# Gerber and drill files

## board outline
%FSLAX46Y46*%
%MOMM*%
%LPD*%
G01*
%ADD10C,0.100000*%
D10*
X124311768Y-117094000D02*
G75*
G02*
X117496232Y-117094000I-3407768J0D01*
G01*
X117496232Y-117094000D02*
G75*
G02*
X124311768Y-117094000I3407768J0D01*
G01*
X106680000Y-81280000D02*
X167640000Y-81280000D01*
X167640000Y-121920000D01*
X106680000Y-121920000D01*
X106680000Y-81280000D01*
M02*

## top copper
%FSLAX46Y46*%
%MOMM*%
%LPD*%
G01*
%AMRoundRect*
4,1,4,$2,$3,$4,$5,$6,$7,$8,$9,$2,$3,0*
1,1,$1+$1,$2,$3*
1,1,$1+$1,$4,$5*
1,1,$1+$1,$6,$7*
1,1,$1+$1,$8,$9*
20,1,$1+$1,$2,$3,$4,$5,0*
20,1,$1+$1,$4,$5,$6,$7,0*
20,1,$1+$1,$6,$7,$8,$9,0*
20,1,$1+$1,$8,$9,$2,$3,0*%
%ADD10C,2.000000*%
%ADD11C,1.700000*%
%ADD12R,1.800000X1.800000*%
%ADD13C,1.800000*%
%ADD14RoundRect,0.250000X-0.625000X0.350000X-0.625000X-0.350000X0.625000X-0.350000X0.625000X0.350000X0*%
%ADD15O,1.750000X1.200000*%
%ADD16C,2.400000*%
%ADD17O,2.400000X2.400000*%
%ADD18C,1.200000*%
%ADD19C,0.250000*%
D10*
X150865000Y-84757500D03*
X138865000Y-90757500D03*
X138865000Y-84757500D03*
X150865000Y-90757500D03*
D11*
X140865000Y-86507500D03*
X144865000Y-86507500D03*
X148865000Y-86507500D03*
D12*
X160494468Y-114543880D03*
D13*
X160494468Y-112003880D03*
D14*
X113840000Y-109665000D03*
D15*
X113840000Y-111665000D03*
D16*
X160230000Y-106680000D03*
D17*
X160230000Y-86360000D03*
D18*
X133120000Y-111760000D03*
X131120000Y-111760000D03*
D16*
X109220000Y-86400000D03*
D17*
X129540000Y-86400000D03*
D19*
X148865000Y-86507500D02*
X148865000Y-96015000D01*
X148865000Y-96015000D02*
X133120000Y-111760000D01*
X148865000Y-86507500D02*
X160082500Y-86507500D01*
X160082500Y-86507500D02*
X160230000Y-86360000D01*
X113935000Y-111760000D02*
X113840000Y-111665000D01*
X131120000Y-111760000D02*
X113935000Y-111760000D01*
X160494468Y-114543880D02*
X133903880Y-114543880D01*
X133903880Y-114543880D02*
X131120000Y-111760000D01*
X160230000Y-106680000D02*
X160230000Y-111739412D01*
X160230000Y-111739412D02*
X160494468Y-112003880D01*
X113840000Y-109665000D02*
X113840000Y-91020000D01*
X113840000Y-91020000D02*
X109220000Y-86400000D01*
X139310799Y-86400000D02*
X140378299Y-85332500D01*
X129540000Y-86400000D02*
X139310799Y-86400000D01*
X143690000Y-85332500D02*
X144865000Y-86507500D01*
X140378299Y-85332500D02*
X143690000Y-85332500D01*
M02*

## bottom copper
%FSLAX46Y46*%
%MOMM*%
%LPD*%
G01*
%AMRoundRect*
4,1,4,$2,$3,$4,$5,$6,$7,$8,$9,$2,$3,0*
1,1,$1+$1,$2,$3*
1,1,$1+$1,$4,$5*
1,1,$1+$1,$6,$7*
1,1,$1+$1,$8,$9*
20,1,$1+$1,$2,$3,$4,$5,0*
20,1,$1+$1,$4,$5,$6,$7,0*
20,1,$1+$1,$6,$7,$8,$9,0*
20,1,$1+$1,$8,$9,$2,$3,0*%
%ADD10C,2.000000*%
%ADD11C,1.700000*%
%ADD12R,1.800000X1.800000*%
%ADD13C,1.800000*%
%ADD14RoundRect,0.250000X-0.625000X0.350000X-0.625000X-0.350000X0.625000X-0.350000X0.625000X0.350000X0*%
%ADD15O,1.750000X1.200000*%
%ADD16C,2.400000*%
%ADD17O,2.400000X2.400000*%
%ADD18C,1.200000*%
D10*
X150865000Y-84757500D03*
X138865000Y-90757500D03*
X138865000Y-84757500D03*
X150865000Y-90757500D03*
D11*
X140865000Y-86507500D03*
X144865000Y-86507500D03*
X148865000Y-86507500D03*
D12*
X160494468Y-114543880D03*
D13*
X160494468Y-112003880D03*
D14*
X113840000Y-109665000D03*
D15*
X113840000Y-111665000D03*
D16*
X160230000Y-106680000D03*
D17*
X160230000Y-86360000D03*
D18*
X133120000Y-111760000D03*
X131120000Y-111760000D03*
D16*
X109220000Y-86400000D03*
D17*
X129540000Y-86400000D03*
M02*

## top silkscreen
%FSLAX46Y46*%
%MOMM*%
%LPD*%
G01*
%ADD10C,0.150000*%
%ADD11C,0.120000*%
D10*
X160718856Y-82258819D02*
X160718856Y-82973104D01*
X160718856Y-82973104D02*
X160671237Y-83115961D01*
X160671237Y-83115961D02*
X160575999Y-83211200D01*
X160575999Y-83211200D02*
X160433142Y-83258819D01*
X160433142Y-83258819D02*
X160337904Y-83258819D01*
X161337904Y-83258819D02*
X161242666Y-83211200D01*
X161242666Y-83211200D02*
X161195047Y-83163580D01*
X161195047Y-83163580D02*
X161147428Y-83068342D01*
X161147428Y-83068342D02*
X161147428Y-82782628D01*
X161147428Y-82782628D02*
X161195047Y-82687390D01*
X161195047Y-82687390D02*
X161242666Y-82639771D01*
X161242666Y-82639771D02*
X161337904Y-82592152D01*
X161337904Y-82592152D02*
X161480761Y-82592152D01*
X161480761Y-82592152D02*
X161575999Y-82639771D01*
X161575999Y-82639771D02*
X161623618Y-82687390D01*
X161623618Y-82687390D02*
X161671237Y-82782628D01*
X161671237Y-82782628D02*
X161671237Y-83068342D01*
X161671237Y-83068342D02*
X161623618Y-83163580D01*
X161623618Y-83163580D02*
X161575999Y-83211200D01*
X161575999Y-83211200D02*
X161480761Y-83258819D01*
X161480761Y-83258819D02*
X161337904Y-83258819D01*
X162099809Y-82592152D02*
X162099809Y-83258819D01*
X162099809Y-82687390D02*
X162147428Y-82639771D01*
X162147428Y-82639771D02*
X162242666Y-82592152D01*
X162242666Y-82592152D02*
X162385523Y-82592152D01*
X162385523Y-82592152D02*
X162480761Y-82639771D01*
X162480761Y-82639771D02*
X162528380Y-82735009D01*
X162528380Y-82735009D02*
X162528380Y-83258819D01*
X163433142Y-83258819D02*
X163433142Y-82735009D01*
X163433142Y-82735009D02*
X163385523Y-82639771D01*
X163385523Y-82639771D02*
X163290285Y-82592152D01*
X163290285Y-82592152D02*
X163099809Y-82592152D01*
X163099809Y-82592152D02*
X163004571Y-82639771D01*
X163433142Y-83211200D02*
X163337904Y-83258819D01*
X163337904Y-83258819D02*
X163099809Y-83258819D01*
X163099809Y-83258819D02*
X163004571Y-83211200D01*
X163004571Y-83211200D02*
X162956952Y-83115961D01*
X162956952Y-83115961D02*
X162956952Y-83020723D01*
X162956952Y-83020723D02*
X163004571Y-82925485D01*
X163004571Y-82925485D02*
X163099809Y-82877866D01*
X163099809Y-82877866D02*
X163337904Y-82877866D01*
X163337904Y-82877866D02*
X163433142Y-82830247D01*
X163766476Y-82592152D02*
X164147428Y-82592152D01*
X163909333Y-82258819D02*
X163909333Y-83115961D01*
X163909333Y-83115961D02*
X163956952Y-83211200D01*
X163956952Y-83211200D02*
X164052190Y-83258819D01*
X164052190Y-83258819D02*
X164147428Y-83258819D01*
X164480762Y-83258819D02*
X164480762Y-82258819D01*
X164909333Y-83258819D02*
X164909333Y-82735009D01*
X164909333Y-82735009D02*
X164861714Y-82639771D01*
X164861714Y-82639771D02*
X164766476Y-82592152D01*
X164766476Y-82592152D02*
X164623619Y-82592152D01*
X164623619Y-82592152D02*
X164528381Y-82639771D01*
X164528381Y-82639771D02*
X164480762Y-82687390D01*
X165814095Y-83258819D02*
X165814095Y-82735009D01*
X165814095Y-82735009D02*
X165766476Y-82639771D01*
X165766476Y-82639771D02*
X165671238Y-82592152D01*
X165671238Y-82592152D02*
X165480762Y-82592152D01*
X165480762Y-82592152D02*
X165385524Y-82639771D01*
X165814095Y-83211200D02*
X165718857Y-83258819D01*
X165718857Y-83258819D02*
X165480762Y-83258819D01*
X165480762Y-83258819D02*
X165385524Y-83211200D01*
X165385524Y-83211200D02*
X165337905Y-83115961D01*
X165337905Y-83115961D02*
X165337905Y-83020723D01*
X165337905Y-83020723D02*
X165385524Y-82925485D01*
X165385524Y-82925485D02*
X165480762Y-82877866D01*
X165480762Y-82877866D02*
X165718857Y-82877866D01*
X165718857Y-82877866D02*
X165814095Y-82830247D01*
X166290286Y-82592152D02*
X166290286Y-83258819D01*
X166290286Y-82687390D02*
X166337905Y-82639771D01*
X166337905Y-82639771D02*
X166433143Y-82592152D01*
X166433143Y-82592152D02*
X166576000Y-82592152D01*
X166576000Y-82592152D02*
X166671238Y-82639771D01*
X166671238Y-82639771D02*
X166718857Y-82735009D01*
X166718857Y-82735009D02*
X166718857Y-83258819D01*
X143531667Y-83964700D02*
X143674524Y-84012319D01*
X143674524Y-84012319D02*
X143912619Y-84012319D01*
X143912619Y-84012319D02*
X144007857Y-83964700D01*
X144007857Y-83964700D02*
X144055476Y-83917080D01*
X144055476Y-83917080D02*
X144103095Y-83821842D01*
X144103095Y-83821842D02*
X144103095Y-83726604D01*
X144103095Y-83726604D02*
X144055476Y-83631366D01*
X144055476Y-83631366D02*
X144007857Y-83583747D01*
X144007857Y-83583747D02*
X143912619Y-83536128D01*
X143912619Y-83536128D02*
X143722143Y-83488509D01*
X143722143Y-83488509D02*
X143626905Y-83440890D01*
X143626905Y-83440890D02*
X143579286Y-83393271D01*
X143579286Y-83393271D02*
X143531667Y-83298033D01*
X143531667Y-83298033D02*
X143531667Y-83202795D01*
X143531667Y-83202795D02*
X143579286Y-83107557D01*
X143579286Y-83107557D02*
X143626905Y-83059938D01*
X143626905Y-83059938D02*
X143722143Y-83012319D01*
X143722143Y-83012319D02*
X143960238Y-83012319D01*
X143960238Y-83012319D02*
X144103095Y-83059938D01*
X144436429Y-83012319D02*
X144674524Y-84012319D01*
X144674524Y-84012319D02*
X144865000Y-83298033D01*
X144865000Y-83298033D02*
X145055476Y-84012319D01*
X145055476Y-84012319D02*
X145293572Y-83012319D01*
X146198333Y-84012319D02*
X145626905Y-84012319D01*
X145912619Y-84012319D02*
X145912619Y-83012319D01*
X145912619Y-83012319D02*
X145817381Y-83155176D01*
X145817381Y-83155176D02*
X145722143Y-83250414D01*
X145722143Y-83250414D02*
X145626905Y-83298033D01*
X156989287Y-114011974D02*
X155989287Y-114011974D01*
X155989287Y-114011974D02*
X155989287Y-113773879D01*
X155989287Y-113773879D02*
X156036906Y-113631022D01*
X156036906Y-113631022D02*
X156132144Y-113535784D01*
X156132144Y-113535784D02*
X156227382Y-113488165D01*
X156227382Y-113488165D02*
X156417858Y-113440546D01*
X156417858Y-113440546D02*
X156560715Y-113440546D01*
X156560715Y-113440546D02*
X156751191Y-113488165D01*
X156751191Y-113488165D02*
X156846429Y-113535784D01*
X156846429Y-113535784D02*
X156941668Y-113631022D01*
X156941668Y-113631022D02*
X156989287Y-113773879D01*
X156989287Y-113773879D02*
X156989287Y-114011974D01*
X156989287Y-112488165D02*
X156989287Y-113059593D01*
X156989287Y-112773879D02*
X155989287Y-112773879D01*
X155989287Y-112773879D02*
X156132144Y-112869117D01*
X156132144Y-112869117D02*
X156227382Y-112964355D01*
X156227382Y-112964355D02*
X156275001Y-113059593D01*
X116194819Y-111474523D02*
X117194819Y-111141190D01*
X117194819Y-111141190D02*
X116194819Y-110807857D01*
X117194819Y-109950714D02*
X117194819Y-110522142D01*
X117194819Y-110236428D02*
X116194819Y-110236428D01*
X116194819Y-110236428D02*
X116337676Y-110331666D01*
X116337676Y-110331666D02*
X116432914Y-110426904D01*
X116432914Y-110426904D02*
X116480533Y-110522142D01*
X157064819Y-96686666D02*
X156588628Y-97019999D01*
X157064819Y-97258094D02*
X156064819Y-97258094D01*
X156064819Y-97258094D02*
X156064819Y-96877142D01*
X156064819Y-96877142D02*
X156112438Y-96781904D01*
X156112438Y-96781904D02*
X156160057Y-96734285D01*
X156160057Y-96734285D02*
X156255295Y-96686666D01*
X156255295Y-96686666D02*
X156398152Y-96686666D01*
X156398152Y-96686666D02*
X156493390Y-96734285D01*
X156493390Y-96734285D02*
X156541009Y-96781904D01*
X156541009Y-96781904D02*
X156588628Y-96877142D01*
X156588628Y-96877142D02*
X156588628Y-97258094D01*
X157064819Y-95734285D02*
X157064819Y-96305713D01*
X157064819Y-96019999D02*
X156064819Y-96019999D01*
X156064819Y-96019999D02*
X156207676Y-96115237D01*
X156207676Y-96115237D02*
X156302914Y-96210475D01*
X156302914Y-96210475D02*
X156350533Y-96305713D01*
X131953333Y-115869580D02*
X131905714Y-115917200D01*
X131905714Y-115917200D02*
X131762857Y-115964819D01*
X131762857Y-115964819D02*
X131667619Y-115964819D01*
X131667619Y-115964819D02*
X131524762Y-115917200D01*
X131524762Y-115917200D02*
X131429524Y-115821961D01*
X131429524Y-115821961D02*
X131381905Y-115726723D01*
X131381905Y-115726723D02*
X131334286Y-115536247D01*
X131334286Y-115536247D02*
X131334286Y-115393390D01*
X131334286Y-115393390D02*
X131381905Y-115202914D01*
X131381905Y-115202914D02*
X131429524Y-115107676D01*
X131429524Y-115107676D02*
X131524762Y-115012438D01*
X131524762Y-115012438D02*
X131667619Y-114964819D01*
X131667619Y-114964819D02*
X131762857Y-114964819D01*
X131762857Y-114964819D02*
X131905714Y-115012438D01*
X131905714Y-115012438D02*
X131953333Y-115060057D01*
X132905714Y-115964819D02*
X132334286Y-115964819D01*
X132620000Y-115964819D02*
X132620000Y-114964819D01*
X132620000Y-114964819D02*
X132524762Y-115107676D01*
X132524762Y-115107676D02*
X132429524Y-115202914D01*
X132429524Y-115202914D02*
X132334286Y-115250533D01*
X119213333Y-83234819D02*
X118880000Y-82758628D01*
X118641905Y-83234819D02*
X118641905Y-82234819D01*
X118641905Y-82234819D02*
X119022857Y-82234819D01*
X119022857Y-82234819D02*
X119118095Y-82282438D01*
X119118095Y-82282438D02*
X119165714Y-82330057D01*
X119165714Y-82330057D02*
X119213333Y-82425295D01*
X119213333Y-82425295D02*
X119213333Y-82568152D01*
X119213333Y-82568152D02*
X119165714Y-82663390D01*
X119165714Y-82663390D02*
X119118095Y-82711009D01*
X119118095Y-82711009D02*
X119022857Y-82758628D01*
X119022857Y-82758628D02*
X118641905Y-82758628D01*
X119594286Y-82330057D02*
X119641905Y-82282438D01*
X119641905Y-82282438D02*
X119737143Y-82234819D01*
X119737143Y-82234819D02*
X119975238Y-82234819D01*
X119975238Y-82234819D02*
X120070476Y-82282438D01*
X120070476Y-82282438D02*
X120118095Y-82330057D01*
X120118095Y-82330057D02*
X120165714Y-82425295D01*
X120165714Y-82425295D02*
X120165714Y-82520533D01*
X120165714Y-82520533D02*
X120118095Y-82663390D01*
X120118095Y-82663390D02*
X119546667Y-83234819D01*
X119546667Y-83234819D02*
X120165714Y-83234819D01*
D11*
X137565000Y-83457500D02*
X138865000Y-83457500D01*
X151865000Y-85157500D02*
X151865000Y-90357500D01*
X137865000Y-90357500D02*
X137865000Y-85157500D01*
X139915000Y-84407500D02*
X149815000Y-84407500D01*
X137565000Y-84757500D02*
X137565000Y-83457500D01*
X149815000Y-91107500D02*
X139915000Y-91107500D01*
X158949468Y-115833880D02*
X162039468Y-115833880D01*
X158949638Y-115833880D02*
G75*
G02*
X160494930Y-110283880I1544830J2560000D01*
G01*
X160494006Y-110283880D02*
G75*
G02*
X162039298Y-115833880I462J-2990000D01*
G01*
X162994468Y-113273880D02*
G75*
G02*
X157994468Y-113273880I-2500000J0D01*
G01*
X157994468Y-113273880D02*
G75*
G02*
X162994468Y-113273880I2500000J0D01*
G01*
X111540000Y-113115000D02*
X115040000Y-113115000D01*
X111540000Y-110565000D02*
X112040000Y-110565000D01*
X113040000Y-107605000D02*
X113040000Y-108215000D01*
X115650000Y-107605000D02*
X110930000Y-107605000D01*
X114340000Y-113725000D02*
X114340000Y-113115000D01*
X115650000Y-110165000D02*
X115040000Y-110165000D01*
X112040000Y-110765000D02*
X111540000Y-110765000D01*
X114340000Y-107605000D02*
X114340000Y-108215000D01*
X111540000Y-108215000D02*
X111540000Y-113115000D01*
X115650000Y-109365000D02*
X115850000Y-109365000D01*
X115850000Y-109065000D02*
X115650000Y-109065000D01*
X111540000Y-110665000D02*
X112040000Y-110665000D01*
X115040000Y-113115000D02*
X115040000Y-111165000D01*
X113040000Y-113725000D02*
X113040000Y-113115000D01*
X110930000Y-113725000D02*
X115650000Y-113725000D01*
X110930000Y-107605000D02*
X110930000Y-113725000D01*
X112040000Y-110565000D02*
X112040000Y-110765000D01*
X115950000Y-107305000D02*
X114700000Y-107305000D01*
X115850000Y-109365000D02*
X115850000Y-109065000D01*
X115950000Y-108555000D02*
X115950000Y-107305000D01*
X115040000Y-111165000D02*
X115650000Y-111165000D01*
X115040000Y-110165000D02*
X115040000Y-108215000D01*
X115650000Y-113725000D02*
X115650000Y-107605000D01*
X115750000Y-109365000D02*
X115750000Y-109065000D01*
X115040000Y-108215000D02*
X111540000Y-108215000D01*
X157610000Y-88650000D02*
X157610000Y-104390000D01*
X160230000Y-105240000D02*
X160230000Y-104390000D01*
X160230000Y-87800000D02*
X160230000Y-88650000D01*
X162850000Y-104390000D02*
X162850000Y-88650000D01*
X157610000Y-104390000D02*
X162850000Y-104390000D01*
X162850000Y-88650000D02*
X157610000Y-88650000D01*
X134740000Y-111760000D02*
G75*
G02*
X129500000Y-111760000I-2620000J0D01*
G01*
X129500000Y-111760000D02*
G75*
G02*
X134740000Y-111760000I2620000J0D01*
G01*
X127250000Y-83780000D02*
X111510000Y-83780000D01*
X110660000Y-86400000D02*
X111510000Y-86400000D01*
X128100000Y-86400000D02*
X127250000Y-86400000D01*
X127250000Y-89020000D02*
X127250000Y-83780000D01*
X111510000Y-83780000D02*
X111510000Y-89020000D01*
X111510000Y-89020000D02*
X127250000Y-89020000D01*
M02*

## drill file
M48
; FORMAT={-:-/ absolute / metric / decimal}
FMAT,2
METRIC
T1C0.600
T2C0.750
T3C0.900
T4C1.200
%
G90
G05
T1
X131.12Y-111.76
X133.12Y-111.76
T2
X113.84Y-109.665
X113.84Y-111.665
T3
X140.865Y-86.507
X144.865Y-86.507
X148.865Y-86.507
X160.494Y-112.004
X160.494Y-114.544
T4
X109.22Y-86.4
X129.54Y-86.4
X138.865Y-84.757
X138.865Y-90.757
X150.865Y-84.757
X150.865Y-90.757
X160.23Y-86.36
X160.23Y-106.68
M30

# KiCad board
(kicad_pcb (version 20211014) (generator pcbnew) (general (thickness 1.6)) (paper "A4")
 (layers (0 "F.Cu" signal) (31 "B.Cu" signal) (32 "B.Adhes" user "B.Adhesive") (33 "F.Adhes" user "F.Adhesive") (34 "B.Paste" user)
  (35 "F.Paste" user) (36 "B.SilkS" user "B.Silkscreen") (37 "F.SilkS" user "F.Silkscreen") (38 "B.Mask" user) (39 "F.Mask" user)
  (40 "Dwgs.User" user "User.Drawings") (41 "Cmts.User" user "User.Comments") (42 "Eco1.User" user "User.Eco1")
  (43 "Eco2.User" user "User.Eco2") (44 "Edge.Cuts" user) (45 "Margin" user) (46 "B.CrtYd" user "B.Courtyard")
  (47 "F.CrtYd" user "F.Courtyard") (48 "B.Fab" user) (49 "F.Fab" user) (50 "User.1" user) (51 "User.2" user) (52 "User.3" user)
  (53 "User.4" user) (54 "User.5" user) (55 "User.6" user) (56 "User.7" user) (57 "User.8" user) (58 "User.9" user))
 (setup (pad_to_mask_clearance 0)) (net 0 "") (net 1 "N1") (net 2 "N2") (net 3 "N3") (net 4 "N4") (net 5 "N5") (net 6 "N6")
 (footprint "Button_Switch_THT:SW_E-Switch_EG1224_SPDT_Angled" (layer "F.Cu") (at 140.865 86.5075)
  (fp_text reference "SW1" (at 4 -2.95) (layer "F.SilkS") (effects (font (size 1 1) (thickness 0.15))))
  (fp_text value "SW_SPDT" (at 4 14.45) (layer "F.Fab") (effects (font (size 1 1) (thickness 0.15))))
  (fp_line (start -3.3 -3.05) (end -2 -3.05) (layer "F.SilkS") (width 0.12))
  (fp_line (start 11 -1.35) (end 11 3.85) (layer "F.SilkS") (width 0.12))
  (fp_line (start -3 3.85) (end -3 -1.35) (layer "F.SilkS") (width 0.12))
  (fp_line (start -0.95 -2.1) (end 8.95 -2.1) (layer "F.SilkS") (width 0.12))
  (fp_line (start -3.3 -1.75) (end -3.3 -3.05) (layer "F.SilkS") (width 0.12))
  (fp_line (start 8.95 4.6) (end -0.95 4.6) (layer "F.SilkS") (width 0.12))
  (pad "" thru_hole circle (at 10 -1.75) (size 2 2) (drill 1.2) (layers *.Cu *.Mask))
  (pad "" thru_hole circle (at -2 4.25) (size 2 2) (drill 1.2) (layers *.Cu *.Mask))
  (pad "" thru_hole circle (at -2 -1.75) (size 2 2) (drill 1.2) (layers *.Cu *.Mask))
  (pad "" thru_hole circle (at 10 4.25) (size 2 2) (drill 1.2) (layers *.Cu *.Mask))
  (pad "1" thru_hole circle (at 0 0) (size 1.7 1.7) (drill 0.9) (layers *.Cu *.Mask) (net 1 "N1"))
  (pad "2" thru_hole circle (at 4 0) (size 1.7 1.7) (drill 0.9) (layers *.Cu *.Mask) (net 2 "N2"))
  (pad "3" thru_hole circle (at 8 0) (size 1.7 1.7) (drill 0.9) (layers *.Cu *.Mask) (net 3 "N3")))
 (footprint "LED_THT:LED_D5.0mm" (layer "F.Cu") (at 160.494468 114.54388 90)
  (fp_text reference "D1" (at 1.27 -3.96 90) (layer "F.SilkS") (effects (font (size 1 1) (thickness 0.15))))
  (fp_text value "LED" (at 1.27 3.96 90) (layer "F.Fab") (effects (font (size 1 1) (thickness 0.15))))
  (fp_line (start -1.29 -1.545) (end -1.29 1.545) (layer "F.SilkS") (width 0.12))
  (fp_arc (start -1.29 -1.54483) (mid 2.072002 -2.880433) (end 4.26 0.000462) (layer "F.SilkS") (width 0.12))
  (fp_arc (start 4.26 -0.000462) (mid 2.072002 2.880433) (end -1.29 1.54483) (layer "F.SilkS") (width 0.12))
  (fp_circle (center 1.27 0) (end 3.77 0) (layer "F.SilkS") (width 0.12) (fill none))
  (pad "1" thru_hole rect (at 0 0 90) (size 1.8 1.8) (drill 0.9) (layers *.Cu *.Mask) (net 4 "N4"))
  (pad "2" thru_hole circle (at 2.54 0 90) (size 1.8 1.8) (drill 0.9) (layers *.Cu *.Mask) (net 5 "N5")))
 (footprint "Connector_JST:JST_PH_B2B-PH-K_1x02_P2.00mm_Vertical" (layer "F.Cu") (at 113.84 109.665 -90)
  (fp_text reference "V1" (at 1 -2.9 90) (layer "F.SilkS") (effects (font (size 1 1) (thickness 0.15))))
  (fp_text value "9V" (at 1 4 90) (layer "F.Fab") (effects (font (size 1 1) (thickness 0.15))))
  (fp_line (start 3.45 2.3) (end 3.45 -1.2) (layer "F.SilkS") (width 0.12))
  (fp_line (start 0.9 2.3) (end 0.9 1.8) (layer "F.SilkS") (width 0.12))
  (fp_line (start -2.06 0.8) (end -1.45 0.8) (layer "F.SilkS") (width 0.12))
  (fp_line (start -2.06 -1.81) (end -2.06 2.91) (layer "F.SilkS") (width 0.12))
  (fp_line (start 4.06 -0.5) (end 3.45 -0.5) (layer "F.SilkS") (width 0.12))
  (fp_line (start 0.5 -1.81) (end 0.5 -1.2) (layer "F.SilkS") (width 0.12))
  (fp_line (start 1.1 1.8) (end 1.1 2.3) (layer "F.SilkS") (width 0.12))
  (fp_line (start -2.06 -0.5) (end -1.45 -0.5) (layer "F.SilkS") (width 0.12))
  (fp_line (start -1.45 2.3) (end 3.45 2.3) (layer "F.SilkS") (width 0.12))
  (fp_line (start -0.3 -1.81) (end -0.3 -2.01) (layer "F.SilkS") (width 0.12))
  (fp_line (start -0.6 -2.01) (end -0.6 -1.81) (layer "F.SilkS") (width 0.12))
  (fp_line (start 1 2.3) (end 1 1.8) (layer "F.SilkS") (width 0.12))
  (fp_line (start 3.45 -1.2) (end 1.5 -1.2) (layer "F.SilkS") (width 0.12))
  (fp_line (start 4.06 0.8) (end 3.45 0.8) (layer "F.SilkS") (width 0.12))
  (fp_line (start 4.06 2.91) (end 4.06 -1.81) (layer "F.SilkS") (width 0.12))
  (fp_line (start -2.06 2.91) (end 4.06 2.91) (layer "F.SilkS") (width 0.12))
  (fp_line (start 0.9 1.8) (end 1.1 1.8) (layer "F.SilkS") (width 0.12))
  (fp_line (start -2.36 -2.11) (end -2.36 -0.86) (layer "F.SilkS") (width 0.12))
  (fp_line (start -0.3 -2.01) (end -0.6 -2.01) (layer "F.SilkS") (width 0.12))
  (fp_line (start -1.11 -2.11) (end -2.36 -2.11) (layer "F.SilkS") (width 0.12))
  (fp_line (start 1.5 -1.2) (end 1.5 -1.81) (layer "F.SilkS") (width 0.12))
  (fp_line (start 0.5 -1.2) (end -1.45 -1.2) (layer "F.SilkS") (width 0.12))
  (fp_line (start 4.06 -1.81) (end -2.06 -1.81) (layer "F.SilkS") (width 0.12))
  (fp_line (start -0.3 -1.91) (end -0.6 -1.91) (layer "F.SilkS") (width 0.12))
  (fp_line (start -1.45 -1.2) (end -1.45 2.3) (layer "F.SilkS") (width 0.12))
  (pad "1" thru_hole roundrect (at 0 0 270) (size 1.2 1.75) (drill 0.75) (layers *.Cu *.Mask) (roundrect_rratio 0.208333) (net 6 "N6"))
  (pad "2" thru_hole oval (at 2 0 270) (size 1.2 1.75) (drill 0.75) (layers *.Cu *.Mask) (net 4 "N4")))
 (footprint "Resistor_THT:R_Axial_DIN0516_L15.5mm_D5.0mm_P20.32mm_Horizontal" (layer "F.Cu") (at 160.23 106.68 90)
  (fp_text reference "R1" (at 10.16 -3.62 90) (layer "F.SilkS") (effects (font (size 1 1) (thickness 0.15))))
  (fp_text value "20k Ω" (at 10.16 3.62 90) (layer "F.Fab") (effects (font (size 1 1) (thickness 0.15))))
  (fp_line (start 18.03 -2.62) (end 2.29 -2.62) (layer "F.SilkS") (width 0.12))
  (fp_line (start 1.44 0) (end 2.29 0) (layer "F.SilkS") (width 0.12))
  (fp_line (start 18.88 0) (end 18.03 0) (layer "F.SilkS") (width 0.12))
  (fp_line (start 2.29 2.62) (end 18.03 2.62) (layer "F.SilkS") (width 0.12))
  (fp_line (start 2.29 -2.62) (end 2.29 2.62) (layer "F.SilkS") (width 0.12))
  (fp_line (start 18.03 2.62) (end 18.03 -2.62) (layer "F.SilkS") (width 0.12))
  (pad "1" thru_hole circle (at 0 0 90) (size 2.4 2.4) (drill 1.2) (layers *.Cu *.Mask) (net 5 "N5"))
  (pad "2" thru_hole oval (at 20.32 0 90) (size 2.4 2.4) (drill 1.2) (layers *.Cu *.Mask) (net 3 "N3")))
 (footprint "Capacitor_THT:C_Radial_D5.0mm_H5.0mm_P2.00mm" (layer "F.Cu") (at 133.12 111.76 180)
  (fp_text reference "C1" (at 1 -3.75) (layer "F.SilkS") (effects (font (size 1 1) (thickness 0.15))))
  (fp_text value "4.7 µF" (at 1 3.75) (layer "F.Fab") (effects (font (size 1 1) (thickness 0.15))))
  (fp_circle (center 1 0) (end 3.62 0) (layer "F.SilkS") (width 0.12) (fill none))
  (pad "1" thru_hole circle (at 0 0 180) (size 1.2 1.2) (drill 0.6) (layers *.Cu *.Mask) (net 3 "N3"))
  (pad "2" thru_hole circle (at 2 0 180) (size 1.2 1.2) (drill 0.6) (layers *.Cu *.Mask) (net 4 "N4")))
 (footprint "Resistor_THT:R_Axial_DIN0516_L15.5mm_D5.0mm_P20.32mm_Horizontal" (layer "F.Cu") (at 109.22 86.4)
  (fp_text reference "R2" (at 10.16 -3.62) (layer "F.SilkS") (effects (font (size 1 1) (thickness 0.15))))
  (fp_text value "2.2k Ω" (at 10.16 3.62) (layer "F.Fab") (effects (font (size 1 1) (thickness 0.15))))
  (fp_line (start 18.03 -2.62) (end 2.29 -2.62) (layer "F.SilkS") (width 0.12))
  (fp_line (start 1.44 0) (end 2.29 0) (layer "F.SilkS") (width 0.12))
  (fp_line (start 18.88 0) (end 18.03 0) (layer "F.SilkS") (width 0.12))
  (fp_line (start 18.03 2.62) (end 18.03 -2.62) (layer "F.SilkS") (width 0.12))
  (fp_line (start 2.29 -2.62) (end 2.29 2.62) (layer "F.SilkS") (width 0.12))
  (fp_line (start 2.29 2.62) (end 18.03 2.62) (layer "F.SilkS") (width 0.12))
  (pad "1" thru_hole circle (at 0 0) (size 2.4 2.4) (drill 1.2) (layers *.Cu *.Mask) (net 6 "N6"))
  (pad "2" thru_hole oval (at 20.32 0) (size 2.4 2.4) (drill 1.2) (layers *.Cu *.Mask) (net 2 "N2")))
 (gr_circle (center 120.904 117.094) (end 122.428 120.142) (layer "Edge.Cuts") (width 0.1) (fill none))
 (gr_rect (start 106.68 81.28) (end 167.64 121.92) (layer "Edge.Cuts") (width 0.1) (fill none))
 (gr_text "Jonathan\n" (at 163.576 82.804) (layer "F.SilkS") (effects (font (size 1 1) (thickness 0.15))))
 (segment (start 148.865 86.5075) (end 148.865 96.015) (width 0.25) (layer "F.Cu") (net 3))
 (segment (start 148.865 96.015) (end 133.12 111.76) (width 0.25) (layer "F.Cu") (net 3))
 (segment (start 148.865 86.5075) (end 160.0825 86.5075) (width 0.25) (layer "F.Cu") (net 3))
 (segment (start 160.0825 86.5075) (end 160.23 86.36) (width 0.25) (layer "F.Cu") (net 3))
 (segment (start 113.935 111.76) (end 113.84 111.665) (width 0.25) (layer "F.Cu") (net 4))
 (segment (start 131.12 111.76) (end 113.935 111.76) (width 0.25) (layer "F.Cu") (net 4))
 (segment (start 160.494468 114.54388) (end 133.90388 114.54388) (width 0.25) (layer "F.Cu") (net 4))
 (segment (start 133.90388 114.54388) (end 131.12 111.76) (width 0.25) (layer "F.Cu") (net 4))
 (segment (start 160.23 106.68) (end 160.23 111.739412) (width 0.25) (layer "F.Cu") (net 5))
 (segment (start 160.23 111.739412) (end 160.494468 112.00388) (width 0.25) (layer "F.Cu") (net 5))
 (segment (start 113.84 109.665) (end 113.84 91.02) (width 0.25) (layer "F.Cu") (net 6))
 (segment (start 113.84 91.02) (end 109.22 86.4) (width 0.25) (layer "F.Cu") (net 6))
 (segment (start 139.310799 86.4) (end 140.378299 85.3325) (width 0.25) (layer "F.Cu") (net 2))
 (segment (start 129.54 86.4) (end 139.310799 86.4) (width 0.25) (layer "F.Cu") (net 2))
 (segment (start 143.69 85.3325) (end 144.865 86.5075) (width 0.25) (layer "F.Cu") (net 2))
 (segment (start 140.378299 85.3325) (end 143.69 85.3325) (width 0.25) (layer "F.Cu") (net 2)))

